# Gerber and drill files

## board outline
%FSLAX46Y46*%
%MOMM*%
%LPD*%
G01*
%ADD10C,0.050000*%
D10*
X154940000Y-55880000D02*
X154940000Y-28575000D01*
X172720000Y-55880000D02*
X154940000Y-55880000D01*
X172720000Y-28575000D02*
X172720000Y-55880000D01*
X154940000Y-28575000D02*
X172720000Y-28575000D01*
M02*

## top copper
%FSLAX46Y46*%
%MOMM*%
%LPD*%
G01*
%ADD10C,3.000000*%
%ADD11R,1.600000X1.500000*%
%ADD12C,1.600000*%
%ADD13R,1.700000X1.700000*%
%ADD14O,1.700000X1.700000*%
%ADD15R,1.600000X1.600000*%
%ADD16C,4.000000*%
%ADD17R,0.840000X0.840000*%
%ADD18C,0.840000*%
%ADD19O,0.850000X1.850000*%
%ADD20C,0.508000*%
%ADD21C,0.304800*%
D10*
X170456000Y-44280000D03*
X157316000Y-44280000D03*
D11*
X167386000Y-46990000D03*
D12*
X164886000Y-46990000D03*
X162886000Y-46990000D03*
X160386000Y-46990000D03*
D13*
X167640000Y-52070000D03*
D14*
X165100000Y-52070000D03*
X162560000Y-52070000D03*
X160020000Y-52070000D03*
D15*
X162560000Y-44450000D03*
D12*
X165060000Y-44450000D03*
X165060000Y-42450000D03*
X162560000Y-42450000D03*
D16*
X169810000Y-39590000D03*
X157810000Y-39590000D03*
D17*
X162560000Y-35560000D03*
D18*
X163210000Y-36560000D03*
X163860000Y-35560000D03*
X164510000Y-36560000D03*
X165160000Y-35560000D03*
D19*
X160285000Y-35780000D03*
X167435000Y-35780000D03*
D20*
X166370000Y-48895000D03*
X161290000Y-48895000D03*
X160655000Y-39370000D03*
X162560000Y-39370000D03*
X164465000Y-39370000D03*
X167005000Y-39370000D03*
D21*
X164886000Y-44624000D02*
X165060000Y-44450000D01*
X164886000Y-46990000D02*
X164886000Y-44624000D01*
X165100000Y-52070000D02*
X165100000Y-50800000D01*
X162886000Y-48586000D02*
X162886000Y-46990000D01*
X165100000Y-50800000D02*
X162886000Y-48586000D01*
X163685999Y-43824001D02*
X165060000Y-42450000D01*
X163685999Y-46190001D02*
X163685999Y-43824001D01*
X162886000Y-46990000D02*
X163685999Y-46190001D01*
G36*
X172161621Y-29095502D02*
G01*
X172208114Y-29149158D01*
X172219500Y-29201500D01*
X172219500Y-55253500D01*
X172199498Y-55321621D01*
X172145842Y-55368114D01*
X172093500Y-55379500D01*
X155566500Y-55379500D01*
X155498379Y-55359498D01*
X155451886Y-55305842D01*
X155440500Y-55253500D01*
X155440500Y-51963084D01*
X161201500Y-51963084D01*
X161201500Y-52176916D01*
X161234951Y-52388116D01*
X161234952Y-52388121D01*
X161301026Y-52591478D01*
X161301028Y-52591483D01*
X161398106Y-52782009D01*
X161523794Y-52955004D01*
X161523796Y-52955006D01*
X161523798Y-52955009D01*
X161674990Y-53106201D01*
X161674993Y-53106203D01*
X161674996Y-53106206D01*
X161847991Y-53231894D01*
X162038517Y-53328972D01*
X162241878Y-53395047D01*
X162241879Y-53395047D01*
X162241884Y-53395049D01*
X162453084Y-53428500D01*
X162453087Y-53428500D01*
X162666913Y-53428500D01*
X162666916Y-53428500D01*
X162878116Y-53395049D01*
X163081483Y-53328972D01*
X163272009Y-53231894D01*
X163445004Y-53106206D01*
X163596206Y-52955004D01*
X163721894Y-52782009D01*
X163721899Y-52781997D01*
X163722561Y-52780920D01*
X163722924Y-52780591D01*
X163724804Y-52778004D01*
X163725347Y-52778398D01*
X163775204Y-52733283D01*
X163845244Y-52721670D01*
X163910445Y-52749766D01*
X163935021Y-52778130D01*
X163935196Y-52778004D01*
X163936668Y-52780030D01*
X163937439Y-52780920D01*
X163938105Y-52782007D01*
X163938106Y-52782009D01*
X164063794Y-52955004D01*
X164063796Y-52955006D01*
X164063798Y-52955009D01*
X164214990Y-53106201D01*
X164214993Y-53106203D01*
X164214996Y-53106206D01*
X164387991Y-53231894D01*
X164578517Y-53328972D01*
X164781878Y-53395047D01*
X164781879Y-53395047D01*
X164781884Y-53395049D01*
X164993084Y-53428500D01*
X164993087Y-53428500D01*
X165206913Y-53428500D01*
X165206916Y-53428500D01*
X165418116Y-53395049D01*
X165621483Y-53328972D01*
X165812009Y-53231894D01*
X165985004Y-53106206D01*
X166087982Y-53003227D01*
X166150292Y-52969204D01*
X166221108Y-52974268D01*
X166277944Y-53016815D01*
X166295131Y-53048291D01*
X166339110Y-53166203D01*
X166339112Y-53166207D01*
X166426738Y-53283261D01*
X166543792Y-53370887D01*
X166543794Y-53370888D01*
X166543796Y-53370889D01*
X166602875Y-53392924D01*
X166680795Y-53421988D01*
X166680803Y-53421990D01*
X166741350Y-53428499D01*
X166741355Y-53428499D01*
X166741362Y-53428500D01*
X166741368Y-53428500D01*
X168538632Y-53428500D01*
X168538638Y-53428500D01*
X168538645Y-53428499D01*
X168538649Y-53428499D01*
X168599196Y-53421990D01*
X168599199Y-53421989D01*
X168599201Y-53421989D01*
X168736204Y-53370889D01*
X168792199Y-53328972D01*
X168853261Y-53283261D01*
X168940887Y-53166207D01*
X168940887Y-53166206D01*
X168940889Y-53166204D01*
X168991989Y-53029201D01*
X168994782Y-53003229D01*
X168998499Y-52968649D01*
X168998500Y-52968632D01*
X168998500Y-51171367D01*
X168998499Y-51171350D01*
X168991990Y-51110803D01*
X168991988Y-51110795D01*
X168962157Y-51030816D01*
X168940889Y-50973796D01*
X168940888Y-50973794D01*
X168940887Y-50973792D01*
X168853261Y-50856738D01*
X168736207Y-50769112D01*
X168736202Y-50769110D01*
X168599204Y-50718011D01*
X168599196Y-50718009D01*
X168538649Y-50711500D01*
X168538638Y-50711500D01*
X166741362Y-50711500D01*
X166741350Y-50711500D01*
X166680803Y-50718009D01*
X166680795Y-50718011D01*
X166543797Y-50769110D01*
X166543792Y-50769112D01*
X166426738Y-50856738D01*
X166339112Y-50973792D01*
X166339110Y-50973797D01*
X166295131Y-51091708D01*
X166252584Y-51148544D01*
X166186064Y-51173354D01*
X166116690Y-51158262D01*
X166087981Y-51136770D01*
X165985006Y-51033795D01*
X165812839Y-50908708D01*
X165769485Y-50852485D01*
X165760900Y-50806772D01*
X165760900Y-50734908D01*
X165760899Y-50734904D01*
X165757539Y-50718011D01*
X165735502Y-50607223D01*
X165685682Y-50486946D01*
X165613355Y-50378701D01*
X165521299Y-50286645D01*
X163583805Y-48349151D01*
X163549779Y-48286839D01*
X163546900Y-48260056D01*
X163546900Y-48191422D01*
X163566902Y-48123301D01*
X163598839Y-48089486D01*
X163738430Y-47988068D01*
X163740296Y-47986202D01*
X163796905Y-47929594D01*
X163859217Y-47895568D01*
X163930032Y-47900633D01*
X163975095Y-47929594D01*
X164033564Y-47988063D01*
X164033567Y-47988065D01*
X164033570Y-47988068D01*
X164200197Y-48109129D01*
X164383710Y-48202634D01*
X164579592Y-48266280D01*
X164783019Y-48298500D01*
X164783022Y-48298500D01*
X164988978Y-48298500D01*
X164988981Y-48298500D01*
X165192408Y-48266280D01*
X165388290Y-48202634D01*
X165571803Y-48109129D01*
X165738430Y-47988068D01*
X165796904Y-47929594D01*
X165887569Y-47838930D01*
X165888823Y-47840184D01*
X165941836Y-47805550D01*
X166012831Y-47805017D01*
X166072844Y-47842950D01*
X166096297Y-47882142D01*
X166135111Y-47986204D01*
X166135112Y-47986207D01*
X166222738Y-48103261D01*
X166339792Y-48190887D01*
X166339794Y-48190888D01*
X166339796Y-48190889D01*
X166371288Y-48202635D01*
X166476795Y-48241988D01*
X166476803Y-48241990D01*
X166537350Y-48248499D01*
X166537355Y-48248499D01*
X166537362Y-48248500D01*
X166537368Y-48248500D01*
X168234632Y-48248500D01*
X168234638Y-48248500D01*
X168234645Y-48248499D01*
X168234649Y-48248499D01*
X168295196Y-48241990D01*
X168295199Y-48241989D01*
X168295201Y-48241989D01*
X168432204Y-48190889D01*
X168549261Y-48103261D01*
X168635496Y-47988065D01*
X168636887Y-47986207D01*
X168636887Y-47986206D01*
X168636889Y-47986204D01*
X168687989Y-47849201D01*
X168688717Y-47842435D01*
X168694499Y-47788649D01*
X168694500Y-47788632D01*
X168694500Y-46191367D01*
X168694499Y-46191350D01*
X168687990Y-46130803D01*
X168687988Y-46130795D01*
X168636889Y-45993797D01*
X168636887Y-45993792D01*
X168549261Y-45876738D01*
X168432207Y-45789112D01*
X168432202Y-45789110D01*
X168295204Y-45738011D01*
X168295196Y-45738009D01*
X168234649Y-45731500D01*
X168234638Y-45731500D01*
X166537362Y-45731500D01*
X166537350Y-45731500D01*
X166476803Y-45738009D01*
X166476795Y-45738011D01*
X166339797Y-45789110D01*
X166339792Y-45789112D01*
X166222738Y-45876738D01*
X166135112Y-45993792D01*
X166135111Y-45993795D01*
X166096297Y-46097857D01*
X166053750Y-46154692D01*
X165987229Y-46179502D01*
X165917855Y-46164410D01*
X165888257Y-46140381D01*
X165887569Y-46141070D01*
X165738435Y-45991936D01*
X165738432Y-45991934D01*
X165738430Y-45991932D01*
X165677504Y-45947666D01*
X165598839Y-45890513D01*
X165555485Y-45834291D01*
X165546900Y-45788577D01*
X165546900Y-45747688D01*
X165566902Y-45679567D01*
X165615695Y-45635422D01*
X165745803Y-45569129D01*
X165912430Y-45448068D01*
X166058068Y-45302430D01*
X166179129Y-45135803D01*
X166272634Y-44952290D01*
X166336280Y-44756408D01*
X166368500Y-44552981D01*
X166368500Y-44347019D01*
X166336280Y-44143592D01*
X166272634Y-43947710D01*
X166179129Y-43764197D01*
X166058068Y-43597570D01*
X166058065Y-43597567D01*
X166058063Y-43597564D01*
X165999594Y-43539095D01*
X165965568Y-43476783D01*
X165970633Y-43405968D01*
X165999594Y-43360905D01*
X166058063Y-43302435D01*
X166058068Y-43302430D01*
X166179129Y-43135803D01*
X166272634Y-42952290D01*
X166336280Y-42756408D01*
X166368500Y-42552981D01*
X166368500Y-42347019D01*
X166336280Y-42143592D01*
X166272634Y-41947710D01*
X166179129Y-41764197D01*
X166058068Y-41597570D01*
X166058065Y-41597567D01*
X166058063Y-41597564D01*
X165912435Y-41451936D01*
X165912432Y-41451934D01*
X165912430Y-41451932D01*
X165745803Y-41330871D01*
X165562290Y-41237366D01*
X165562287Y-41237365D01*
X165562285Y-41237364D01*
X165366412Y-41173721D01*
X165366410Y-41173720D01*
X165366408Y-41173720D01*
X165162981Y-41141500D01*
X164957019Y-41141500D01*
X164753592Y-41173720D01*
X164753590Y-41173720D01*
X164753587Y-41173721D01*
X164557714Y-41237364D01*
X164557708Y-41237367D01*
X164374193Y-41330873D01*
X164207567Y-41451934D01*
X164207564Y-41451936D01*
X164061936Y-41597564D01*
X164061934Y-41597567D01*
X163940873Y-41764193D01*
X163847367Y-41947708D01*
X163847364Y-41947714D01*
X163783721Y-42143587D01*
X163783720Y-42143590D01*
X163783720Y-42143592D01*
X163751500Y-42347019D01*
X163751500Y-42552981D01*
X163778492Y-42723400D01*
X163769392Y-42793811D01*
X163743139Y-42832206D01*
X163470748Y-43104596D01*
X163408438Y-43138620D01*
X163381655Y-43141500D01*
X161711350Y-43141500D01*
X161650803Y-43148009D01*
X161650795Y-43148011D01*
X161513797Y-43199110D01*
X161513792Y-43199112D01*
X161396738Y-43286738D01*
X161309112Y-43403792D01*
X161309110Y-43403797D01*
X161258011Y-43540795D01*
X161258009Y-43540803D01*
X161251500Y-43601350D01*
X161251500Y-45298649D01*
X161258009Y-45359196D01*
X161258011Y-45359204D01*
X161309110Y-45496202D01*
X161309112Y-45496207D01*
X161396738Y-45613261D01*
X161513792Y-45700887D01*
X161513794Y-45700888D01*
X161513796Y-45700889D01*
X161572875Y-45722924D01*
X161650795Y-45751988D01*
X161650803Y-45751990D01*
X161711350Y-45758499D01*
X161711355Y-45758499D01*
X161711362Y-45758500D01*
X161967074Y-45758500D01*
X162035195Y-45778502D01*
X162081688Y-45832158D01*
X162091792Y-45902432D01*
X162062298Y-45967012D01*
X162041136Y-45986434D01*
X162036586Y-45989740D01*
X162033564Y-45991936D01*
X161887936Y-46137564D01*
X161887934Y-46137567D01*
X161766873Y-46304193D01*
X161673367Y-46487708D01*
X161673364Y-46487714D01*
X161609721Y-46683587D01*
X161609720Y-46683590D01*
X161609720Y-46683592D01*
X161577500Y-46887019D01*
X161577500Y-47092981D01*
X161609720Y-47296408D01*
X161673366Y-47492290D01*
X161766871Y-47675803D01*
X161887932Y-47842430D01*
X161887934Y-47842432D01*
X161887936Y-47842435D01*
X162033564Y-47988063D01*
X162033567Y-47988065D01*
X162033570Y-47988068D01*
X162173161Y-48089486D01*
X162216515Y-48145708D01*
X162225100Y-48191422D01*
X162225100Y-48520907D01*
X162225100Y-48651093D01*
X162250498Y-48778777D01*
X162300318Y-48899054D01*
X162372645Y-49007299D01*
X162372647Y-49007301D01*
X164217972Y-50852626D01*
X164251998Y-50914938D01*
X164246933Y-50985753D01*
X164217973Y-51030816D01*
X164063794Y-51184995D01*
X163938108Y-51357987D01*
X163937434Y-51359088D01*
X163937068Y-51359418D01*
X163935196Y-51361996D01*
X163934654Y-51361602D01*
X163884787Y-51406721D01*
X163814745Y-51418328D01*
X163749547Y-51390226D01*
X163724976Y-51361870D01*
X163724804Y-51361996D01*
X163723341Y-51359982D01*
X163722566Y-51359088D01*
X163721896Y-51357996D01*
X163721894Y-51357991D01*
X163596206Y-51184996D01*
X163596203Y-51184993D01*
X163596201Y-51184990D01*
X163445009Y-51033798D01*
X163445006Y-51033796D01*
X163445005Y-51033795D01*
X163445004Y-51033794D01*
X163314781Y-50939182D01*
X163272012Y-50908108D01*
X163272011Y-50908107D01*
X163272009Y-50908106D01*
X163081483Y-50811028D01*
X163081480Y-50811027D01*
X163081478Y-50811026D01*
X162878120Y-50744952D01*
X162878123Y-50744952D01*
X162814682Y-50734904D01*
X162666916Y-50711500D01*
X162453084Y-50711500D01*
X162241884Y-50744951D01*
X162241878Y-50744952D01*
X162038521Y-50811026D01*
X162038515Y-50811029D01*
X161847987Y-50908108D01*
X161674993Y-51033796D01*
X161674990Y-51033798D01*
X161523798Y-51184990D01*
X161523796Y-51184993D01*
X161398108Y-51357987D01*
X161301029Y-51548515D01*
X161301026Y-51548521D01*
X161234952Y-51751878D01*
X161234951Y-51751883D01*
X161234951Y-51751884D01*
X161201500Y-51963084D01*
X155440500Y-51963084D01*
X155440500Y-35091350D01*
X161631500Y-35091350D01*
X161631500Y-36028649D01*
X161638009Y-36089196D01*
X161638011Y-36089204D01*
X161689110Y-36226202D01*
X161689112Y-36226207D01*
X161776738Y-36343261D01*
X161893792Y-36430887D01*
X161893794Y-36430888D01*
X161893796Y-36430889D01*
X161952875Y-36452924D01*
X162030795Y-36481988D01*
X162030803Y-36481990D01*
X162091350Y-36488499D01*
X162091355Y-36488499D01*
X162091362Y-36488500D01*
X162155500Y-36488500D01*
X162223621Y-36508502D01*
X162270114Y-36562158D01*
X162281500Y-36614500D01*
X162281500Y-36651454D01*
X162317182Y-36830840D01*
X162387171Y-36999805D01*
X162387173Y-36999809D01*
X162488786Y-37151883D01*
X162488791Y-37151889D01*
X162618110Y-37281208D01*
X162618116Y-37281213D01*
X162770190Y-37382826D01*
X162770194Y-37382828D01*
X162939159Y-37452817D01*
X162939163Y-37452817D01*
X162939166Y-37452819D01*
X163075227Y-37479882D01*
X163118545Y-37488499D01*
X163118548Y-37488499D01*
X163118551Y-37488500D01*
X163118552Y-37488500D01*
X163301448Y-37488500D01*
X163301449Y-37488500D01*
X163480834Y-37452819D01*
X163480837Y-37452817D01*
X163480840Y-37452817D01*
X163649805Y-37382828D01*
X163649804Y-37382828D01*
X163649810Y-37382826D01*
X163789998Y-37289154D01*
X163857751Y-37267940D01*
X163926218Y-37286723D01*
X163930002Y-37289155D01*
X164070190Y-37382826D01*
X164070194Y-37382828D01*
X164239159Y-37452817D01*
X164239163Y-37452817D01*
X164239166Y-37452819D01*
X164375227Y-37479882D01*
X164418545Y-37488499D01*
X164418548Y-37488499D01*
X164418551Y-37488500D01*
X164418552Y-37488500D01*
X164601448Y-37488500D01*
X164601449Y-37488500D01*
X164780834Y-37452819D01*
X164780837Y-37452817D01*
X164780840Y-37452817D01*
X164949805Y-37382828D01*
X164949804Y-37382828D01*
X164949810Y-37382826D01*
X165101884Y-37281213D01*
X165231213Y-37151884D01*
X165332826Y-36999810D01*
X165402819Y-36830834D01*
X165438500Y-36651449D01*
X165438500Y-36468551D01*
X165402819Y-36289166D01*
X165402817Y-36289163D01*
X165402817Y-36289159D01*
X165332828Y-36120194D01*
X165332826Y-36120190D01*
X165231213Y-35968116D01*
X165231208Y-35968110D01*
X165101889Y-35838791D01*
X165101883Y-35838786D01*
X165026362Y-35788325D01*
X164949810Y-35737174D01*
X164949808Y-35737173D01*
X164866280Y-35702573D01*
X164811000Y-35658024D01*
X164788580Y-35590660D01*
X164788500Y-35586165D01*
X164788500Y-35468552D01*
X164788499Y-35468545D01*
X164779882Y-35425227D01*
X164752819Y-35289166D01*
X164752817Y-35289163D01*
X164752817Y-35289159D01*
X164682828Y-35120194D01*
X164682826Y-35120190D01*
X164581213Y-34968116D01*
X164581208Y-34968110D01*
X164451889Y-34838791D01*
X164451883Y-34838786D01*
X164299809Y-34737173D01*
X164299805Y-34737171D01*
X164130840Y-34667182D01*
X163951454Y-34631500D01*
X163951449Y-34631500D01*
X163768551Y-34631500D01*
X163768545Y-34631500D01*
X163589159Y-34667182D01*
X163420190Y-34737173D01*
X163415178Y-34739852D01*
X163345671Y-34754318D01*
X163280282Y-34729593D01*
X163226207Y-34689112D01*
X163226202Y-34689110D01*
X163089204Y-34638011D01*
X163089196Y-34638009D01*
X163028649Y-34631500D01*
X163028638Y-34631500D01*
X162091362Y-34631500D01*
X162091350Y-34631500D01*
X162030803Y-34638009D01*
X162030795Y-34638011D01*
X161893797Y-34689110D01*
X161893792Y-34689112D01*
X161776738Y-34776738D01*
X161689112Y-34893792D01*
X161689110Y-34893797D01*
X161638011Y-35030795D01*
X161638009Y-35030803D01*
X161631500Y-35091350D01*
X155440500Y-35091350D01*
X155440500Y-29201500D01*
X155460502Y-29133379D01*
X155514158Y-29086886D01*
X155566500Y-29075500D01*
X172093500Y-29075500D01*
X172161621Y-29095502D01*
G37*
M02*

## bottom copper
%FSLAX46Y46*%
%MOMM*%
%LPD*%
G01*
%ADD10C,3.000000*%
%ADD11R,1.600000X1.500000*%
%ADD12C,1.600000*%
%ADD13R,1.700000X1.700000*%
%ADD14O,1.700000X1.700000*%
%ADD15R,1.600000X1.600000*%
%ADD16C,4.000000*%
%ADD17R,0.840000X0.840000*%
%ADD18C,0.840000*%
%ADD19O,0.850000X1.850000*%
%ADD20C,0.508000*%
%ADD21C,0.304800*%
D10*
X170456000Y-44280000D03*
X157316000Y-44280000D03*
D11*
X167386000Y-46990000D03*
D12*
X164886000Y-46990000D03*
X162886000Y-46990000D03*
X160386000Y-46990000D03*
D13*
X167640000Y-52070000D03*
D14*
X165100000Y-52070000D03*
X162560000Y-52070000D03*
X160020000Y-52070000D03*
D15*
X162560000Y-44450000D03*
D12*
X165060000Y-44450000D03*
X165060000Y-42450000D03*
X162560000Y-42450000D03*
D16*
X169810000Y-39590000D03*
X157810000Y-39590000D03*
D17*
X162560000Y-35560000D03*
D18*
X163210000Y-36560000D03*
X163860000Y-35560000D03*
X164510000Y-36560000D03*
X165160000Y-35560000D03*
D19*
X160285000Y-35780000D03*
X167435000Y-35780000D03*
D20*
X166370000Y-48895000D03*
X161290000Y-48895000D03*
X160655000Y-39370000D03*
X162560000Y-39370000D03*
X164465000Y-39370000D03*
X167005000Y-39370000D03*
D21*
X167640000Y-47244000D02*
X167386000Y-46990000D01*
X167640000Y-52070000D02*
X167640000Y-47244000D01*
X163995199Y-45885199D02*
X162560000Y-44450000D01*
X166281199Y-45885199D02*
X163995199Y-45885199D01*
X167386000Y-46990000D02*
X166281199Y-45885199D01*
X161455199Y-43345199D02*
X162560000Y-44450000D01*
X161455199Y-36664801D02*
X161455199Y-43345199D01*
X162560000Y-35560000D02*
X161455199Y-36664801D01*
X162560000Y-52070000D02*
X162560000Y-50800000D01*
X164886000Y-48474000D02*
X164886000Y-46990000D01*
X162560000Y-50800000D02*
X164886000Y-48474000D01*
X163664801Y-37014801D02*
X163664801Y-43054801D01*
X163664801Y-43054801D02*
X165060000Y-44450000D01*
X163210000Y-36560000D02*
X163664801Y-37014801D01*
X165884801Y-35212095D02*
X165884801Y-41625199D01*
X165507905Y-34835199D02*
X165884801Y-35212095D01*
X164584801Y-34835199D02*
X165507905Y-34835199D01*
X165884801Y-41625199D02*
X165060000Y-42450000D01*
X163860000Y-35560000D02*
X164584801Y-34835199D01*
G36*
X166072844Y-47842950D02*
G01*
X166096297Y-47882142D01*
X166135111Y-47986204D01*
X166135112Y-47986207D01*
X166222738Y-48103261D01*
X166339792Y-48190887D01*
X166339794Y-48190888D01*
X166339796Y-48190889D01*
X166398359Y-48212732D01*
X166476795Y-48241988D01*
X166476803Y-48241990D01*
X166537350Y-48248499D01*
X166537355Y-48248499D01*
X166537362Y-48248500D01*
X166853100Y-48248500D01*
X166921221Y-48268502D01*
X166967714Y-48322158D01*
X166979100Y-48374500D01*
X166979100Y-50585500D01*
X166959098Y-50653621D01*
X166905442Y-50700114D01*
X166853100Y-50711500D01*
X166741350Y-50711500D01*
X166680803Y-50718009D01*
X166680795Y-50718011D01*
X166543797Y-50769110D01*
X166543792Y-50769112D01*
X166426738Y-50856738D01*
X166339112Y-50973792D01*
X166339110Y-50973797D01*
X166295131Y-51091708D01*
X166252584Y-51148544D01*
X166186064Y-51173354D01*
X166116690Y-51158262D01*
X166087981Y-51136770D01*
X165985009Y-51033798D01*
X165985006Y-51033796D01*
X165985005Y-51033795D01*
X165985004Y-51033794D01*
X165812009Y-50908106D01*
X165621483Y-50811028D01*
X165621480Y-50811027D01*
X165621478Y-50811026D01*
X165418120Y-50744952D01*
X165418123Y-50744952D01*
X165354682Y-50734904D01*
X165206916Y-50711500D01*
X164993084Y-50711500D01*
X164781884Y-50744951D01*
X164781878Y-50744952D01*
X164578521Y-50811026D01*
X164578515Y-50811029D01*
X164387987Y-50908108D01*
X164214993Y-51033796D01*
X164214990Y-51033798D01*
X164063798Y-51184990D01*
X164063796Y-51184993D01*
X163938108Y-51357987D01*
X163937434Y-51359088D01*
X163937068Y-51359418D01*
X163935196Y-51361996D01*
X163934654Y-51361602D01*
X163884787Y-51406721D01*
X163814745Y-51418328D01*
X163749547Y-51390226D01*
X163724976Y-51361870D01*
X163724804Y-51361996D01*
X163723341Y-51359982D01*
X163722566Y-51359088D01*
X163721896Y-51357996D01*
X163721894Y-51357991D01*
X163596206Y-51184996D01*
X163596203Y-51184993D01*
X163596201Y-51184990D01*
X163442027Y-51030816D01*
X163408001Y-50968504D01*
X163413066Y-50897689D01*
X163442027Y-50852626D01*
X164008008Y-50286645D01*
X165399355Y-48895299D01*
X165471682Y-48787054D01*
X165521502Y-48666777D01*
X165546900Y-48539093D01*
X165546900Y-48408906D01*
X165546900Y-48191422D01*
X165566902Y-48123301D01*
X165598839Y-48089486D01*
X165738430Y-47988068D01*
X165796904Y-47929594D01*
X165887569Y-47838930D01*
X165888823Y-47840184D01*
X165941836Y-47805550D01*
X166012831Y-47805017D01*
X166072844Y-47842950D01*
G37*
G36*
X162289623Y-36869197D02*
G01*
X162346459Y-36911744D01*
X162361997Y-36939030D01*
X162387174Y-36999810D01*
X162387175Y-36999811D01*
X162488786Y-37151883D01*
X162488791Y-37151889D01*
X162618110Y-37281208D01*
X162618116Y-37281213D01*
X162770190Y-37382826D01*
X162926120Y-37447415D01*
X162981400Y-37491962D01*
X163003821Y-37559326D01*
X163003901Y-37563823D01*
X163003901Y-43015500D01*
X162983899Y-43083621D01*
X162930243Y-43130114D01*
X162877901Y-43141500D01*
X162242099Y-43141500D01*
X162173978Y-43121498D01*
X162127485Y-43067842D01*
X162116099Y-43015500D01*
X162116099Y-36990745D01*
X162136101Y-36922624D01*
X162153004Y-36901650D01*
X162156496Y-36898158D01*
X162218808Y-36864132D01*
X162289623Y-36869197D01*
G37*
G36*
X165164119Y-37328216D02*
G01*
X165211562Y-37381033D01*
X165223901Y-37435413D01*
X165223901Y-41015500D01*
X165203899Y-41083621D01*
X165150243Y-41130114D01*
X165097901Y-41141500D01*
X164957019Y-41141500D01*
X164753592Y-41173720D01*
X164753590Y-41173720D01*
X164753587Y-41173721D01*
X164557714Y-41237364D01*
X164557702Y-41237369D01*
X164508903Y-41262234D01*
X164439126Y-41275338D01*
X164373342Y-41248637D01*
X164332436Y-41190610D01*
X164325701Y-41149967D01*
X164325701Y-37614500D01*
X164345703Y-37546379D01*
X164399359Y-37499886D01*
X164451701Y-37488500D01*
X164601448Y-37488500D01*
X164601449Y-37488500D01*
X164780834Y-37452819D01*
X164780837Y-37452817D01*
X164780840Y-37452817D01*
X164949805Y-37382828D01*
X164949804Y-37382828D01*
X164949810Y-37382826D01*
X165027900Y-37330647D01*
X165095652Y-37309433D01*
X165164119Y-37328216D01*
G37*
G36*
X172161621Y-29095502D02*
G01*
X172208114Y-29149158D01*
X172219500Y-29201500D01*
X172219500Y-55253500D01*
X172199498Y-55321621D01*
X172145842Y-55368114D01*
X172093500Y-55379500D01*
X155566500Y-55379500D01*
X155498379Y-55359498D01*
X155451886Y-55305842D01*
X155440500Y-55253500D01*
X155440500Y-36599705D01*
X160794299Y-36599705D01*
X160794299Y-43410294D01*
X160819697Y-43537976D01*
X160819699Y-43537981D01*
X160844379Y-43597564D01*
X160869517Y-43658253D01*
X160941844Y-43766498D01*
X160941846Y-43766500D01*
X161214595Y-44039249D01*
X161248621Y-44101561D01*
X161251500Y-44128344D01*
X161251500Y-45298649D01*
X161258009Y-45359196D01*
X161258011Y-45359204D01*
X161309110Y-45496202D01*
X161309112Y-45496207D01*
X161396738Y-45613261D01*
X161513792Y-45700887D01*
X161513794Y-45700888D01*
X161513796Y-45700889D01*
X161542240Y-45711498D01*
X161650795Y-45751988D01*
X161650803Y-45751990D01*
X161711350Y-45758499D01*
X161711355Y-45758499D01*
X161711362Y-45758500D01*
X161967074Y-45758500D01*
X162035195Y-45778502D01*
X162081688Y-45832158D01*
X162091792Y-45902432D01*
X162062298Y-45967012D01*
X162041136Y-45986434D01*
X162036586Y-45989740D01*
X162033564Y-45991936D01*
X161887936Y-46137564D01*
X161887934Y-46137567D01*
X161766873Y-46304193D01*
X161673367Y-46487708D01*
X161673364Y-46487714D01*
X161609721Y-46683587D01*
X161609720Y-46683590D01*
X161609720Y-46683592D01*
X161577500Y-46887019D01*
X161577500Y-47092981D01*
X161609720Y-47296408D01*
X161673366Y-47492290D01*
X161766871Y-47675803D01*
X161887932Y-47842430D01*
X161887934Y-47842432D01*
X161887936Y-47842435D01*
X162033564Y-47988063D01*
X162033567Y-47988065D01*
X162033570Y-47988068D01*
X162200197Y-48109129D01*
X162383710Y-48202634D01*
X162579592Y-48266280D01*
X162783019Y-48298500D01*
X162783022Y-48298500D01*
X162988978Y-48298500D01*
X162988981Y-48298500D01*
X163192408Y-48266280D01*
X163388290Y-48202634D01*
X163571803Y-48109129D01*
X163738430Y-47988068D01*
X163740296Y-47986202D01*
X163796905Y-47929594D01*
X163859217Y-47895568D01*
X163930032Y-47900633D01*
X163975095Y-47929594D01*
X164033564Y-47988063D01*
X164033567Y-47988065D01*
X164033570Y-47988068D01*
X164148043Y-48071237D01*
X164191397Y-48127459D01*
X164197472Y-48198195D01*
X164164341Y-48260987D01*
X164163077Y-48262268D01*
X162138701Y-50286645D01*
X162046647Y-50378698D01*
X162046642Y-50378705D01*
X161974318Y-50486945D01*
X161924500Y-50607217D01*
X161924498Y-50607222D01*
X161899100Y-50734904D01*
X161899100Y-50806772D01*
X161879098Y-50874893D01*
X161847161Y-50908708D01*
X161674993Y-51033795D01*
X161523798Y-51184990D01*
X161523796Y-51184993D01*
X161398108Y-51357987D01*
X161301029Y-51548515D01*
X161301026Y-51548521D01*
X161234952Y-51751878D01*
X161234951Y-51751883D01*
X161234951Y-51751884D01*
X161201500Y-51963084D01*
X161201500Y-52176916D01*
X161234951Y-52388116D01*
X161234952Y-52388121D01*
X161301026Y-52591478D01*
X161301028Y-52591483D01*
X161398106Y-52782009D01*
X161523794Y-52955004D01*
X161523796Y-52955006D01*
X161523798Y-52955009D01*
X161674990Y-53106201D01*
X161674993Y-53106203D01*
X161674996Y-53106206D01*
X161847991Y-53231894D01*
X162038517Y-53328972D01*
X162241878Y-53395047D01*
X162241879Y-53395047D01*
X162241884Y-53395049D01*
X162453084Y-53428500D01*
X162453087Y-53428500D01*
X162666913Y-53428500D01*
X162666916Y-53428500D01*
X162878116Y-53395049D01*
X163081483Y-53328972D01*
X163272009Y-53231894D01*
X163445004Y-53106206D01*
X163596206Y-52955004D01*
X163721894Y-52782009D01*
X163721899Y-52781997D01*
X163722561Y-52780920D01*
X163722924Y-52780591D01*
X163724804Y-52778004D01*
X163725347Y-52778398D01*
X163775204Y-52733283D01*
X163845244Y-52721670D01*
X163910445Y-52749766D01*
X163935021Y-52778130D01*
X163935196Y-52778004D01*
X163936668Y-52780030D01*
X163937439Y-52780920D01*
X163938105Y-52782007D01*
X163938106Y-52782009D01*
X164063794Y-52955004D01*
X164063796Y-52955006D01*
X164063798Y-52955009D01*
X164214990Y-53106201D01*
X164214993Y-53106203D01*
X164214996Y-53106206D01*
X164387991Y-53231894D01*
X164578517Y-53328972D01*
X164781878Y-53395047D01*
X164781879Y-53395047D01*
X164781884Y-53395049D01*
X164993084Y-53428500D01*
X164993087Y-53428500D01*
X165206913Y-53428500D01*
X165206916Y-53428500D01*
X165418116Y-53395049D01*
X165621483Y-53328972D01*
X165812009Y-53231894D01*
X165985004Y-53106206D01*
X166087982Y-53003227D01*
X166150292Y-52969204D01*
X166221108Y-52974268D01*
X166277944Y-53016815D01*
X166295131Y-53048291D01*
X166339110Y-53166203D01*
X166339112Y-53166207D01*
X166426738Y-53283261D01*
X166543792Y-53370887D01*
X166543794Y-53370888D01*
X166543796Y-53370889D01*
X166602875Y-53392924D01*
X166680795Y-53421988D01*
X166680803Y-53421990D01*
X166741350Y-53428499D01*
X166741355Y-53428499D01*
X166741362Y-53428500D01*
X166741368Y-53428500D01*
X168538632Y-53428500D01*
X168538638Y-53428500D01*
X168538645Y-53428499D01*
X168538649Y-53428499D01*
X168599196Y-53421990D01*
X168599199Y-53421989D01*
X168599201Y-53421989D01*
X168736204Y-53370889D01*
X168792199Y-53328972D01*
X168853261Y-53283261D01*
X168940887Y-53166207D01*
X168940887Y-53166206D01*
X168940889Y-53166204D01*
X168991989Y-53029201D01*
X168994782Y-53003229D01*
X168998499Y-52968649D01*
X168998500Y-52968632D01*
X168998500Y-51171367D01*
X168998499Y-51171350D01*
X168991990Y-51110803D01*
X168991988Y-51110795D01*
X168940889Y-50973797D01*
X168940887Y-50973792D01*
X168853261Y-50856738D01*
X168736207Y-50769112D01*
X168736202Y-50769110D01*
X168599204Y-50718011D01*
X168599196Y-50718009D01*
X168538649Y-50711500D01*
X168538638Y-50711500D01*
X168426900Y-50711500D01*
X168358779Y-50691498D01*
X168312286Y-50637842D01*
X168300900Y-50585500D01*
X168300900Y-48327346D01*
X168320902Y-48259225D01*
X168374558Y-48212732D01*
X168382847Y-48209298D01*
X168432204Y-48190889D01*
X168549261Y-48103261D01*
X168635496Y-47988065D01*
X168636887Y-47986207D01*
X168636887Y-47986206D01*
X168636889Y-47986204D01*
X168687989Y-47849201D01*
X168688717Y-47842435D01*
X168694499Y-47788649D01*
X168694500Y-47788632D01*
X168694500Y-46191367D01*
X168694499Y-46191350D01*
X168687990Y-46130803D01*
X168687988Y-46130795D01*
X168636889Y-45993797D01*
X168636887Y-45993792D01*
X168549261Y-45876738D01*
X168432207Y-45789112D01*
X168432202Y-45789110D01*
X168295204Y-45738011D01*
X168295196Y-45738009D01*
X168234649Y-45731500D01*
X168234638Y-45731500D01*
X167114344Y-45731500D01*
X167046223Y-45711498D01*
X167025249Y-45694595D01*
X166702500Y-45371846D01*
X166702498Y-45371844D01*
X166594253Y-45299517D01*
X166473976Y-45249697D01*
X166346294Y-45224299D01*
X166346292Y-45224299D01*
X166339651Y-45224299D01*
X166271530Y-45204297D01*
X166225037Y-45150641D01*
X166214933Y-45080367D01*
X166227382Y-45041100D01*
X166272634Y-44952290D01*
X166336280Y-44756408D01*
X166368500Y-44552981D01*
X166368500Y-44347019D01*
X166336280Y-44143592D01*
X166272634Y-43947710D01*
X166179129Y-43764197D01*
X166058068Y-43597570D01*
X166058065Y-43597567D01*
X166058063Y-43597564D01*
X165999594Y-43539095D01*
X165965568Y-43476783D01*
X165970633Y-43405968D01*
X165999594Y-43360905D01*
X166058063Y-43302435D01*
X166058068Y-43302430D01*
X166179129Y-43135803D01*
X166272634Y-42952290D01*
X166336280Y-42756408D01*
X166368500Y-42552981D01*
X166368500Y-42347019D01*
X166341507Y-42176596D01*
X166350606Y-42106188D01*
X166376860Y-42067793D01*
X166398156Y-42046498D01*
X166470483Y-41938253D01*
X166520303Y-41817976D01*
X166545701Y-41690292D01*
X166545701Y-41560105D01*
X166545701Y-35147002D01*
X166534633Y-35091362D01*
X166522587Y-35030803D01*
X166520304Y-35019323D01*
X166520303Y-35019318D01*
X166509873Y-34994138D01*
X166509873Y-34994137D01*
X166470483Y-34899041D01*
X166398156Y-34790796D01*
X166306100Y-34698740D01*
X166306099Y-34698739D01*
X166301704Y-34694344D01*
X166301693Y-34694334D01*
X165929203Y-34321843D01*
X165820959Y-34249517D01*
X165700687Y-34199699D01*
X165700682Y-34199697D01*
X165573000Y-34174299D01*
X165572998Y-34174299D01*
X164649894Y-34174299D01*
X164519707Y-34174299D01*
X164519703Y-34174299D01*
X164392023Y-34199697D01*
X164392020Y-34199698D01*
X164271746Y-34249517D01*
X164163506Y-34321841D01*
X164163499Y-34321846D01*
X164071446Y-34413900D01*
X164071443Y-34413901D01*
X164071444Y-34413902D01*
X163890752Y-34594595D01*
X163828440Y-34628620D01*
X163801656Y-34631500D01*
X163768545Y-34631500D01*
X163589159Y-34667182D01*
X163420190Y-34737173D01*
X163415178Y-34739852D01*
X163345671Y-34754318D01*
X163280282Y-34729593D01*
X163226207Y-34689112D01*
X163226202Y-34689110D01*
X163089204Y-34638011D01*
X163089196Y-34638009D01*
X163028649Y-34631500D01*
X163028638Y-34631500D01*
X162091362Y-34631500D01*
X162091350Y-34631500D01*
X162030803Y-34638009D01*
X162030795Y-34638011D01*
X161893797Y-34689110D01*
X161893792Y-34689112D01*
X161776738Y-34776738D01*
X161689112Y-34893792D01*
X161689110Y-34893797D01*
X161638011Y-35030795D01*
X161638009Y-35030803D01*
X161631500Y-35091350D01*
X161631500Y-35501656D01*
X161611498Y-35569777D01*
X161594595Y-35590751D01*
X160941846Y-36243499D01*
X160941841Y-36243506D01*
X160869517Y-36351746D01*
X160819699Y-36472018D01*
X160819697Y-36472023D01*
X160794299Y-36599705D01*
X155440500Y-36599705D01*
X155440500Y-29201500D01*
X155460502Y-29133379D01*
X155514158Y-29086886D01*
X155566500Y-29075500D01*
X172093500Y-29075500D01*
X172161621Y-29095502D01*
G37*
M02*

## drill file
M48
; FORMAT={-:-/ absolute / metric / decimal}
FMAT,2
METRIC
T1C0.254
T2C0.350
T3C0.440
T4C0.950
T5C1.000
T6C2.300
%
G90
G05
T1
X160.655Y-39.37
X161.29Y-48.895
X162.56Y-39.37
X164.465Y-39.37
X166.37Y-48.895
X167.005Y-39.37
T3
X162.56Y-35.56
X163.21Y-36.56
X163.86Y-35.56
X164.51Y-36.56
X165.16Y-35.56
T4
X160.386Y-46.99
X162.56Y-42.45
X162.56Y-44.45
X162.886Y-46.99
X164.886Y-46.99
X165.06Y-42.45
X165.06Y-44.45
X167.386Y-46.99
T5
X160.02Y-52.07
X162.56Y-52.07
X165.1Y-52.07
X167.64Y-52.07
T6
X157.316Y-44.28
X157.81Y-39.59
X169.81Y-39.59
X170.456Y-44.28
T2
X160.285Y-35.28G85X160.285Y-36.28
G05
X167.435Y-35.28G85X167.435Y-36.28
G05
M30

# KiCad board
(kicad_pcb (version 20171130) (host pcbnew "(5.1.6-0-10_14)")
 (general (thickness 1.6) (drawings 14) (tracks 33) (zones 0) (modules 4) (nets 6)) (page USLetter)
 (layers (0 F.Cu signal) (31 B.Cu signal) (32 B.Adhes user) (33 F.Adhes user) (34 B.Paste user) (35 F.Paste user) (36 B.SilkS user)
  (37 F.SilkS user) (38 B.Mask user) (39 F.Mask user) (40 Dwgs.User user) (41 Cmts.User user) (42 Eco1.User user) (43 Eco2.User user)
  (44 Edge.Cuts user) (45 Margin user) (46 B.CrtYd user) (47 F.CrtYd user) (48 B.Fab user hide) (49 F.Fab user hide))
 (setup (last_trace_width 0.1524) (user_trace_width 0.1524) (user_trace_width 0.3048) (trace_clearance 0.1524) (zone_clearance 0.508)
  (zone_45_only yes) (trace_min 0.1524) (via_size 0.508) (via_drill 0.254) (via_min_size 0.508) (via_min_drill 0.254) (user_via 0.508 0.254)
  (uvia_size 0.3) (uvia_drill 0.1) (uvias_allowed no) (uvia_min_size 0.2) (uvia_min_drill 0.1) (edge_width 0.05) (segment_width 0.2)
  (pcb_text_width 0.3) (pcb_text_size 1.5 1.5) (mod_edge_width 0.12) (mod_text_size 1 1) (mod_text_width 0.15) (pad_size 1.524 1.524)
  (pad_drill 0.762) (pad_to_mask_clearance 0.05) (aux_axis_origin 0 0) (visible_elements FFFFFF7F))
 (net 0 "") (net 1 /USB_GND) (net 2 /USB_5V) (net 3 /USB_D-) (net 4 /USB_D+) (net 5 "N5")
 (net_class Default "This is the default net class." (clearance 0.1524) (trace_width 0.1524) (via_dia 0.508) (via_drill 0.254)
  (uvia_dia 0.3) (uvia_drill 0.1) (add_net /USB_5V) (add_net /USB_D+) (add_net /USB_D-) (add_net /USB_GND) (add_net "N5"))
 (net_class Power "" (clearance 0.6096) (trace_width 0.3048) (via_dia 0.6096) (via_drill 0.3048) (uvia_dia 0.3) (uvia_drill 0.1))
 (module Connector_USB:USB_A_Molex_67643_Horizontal (layer F.Cu) (at 167.386 46.99 180)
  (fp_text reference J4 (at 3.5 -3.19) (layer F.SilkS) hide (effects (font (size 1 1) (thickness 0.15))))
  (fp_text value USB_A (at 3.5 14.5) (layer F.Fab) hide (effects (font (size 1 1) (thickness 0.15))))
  (pad 5 thru_hole circle (at -3.07 2.71 180) (size 3 3) (drill 2.3) (layers *.Cu *.Mask) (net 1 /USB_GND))
  (pad 5 thru_hole circle (at 10.07 2.71 180) (size 3 3) (drill 2.3) (layers *.Cu *.Mask) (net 1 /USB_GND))
  (pad 1 thru_hole rect (at 0 0 180) (size 1.6 1.5) (drill 0.95) (layers *.Cu *.Mask) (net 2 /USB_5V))
  (pad 2 thru_hole circle (at 2.5 0 180) (size 1.6 1.6) (drill 0.95) (layers *.Cu *.Mask) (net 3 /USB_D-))
  (pad 3 thru_hole circle (at 4.5 0 180) (size 1.6 1.6) (drill 0.95) (layers *.Cu *.Mask) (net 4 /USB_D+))
  (pad 4 thru_hole circle (at 7 0 180) (size 1.6 1.6) (drill 0.95) (layers *.Cu *.Mask) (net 1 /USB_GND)))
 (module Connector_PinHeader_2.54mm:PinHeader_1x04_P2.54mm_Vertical (layer F.Cu) (at 167.64 52.07 270)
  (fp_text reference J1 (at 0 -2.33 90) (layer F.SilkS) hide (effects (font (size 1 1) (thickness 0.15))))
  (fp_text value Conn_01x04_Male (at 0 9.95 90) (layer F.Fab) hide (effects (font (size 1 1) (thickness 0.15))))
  (pad 1 thru_hole rect (at 0 0 270) (size 1.7 1.7) (drill 1) (layers *.Cu *.Mask) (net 2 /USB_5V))
  (pad 2 thru_hole oval (at 0 2.54 270) (size 1.7 1.7) (drill 1) (layers *.Cu *.Mask) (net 4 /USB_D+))
  (pad 3 thru_hole oval (at 0 5.08 270) (size 1.7 1.7) (drill 1) (layers *.Cu *.Mask) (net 3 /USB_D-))
  (pad 4 thru_hole oval (at 0 7.62 270) (size 1.7 1.7) (drill 1) (layers *.Cu *.Mask) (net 1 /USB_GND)))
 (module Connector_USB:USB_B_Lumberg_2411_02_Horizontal (layer F.Cu) (at 162.56 44.45 90)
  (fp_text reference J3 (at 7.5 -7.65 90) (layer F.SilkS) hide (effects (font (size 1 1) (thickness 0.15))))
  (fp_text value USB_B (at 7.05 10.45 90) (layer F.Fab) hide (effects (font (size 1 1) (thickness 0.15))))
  (pad 1 thru_hole rect (at 0 0 180) (size 1.6 1.6) (drill 0.95) (layers *.Cu *.Mask) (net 2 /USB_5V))
  (pad 2 thru_hole circle (at 0 2.5 180) (size 1.6 1.6) (drill 0.95) (layers *.Cu *.Mask) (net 3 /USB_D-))
  (pad 3 thru_hole circle (at 2 2.5 180) (size 1.6 1.6) (drill 0.95) (layers *.Cu *.Mask) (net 4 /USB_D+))
  (pad 4 thru_hole circle (at 2 0 180) (size 1.6 1.6) (drill 0.95) (layers *.Cu *.Mask) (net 1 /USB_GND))
  (pad 5 thru_hole circle (at 4.86 7.25 180) (size 4 4) (drill 2.3) (layers *.Cu *.Mask) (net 1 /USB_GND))
  (pad 5 thru_hole circle (at 4.86 -4.75 180) (size 4 4) (drill 2.3) (layers *.Cu *.Mask) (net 1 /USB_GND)))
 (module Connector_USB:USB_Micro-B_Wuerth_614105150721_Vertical (layer F.Cu) (at 162.56 35.56)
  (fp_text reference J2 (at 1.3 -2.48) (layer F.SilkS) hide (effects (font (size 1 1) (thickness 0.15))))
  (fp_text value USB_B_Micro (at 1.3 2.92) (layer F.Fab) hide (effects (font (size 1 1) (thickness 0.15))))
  (pad 1 thru_hole rect (at 0 0) (size 0.84 0.84) (drill 0.44) (layers *.Cu *.Mask) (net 2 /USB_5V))
  (pad 2 thru_hole circle (at 0.65 1) (size 0.84 0.84) (drill 0.44) (layers *.Cu *.Mask) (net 3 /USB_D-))
  (pad 3 thru_hole circle (at 1.3 0) (size 0.84 0.84) (drill 0.44) (layers *.Cu *.Mask) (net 4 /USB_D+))
  (pad 4 thru_hole circle (at 1.95 1) (size 0.84 0.84) (drill 0.44) (layers *.Cu *.Mask) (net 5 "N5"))
  (pad 5 thru_hole circle (at 2.6 0) (size 0.84 0.84) (drill 0.44) (layers *.Cu *.Mask) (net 1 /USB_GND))
  (pad 6 thru_hole oval (at -2.275 0.22) (size 0.85 1.85) (drill oval 0.35 1.35) (layers *.Cu *.Mask) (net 1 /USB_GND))
  (pad 6 thru_hole oval (at 4.875 0.22) (size 0.85 1.85) (drill oval 0.35 1.35) (layers *.Cu *.Mask) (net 1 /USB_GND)))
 (gr_line (start 154.94 55.88) (end 154.94 28.575) (layer Edge.Cuts) (width 0.05))
 (gr_line (start 172.72 55.88) (end 154.94 55.88) (layer Edge.Cuts) (width 0.05))
 (gr_line (start 172.72 28.575) (end 172.72 55.88) (layer Edge.Cuts) (width 0.05))
 (gr_line (start 154.94 28.575) (end 172.72 28.575) (layer Edge.Cuts) (width 0.05))
 (via (at 166.37 48.895) (size 0.508) (drill 0.254) (layers F.Cu B.Cu) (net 1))
 (via (at 161.29 48.895) (size 0.508) (drill 0.254) (layers F.Cu B.Cu) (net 1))
 (via (at 160.655 39.37) (size 0.508) (drill 0.254) (layers F.Cu B.Cu) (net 1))
 (via (at 162.56 39.37) (size 0.508) (drill 0.254) (layers F.Cu B.Cu) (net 1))
 (via (at 164.465 39.37) (size 0.508) (drill 0.254) (layers F.Cu B.Cu) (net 1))
 (via (at 167.005 39.37) (size 0.508) (drill 0.254) (layers F.Cu B.Cu) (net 1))
 (segment (start 167.64 47.244) (end 167.386 46.99) (width 0.3048) (layer B.Cu) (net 2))
 (segment (start 167.64 52.07) (end 167.64 47.244) (width 0.3048) (layer B.Cu) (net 2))
 (segment (start 163.995199 45.885199) (end 162.56 44.45) (width 0.3048) (layer B.Cu) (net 2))
 (segment (start 166.281199 45.885199) (end 163.995199 45.885199) (width 0.3048) (layer B.Cu) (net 2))
 (segment (start 167.386 46.99) (end 166.281199 45.885199) (width 0.3048) (layer B.Cu) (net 2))
 (segment (start 161.455199 43.345199) (end 162.56 44.45) (width 0.3048) (layer B.Cu) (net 2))
 (segment (start 161.455199 36.664801) (end 161.455199 43.345199) (width 0.3048) (layer B.Cu) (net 2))
 (segment (start 162.56 35.56) (end 161.455199 36.664801) (width 0.3048) (layer B.Cu) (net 2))
 (segment (start 162.56 52.07) (end 162.56 50.8) (width 0.3048) (layer B.Cu) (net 3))
 (segment (start 164.886 48.474) (end 164.886 46.99) (width 0.3048) (layer B.Cu) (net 3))
 (segment (start 162.56 50.8) (end 164.886 48.474) (width 0.3048) (layer B.Cu) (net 3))
 (segment (start 163.664801 37.014801) (end 163.664801 43.054801) (width 0.3048) (layer B.Cu) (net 3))
 (segment (start 163.664801 43.054801) (end 165.06 44.45) (width 0.3048) (layer B.Cu) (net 3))
 (segment (start 163.21 36.56) (end 163.664801 37.014801) (width 0.3048) (layer B.Cu) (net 3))
 (segment (start 164.886 44.624) (end 165.06 44.45) (width 0.3048) (layer F.Cu) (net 3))
 (segment (start 164.886 46.99) (end 164.886 44.624) (width 0.3048) (layer F.Cu) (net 3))
 (segment (start 165.884801 35.212095) (end 165.884801 41.625199) (width 0.3048) (layer B.Cu) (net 4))
 (segment (start 165.507905 34.835199) (end 165.884801 35.212095) (width 0.3048) (layer B.Cu) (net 4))
 (segment (start 164.584801 34.835199) (end 165.507905 34.835199) (width 0.3048) (layer B.Cu) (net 4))
 (segment (start 165.884801 41.625199) (end 165.06 42.45) (width 0.3048) (layer B.Cu) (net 4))
 (segment (start 163.86 35.56) (end 164.584801 34.835199) (width 0.3048) (layer B.Cu) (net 4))
 (segment (start 165.1 52.07) (end 165.1 50.8) (width 0.3048) (layer F.Cu) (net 4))
 (segment (start 162.886 48.586) (end 162.886 46.99) (width 0.3048) (layer F.Cu) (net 4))
 (segment (start 165.1 50.8) (end 162.886 48.586) (width 0.3048) (layer F.Cu) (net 4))
 (segment (start 163.685999 43.824001) (end 165.06 42.45) (width 0.3048) (layer F.Cu) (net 4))
 (segment (start 163.685999 46.190001) (end 163.685999 43.824001) (width 0.3048) (layer F.Cu) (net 4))
 (segment (start 162.886 46.99) (end 163.685999 46.190001) (width 0.3048) (layer F.Cu) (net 4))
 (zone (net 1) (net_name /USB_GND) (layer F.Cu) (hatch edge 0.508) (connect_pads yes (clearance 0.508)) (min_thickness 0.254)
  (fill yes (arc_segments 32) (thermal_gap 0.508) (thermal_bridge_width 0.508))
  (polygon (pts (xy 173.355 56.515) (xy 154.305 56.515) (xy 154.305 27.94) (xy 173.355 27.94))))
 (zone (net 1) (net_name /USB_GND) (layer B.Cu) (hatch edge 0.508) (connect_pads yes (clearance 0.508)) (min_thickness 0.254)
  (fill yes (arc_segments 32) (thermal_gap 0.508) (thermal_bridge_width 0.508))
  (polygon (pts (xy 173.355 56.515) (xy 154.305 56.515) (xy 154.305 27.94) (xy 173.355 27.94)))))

